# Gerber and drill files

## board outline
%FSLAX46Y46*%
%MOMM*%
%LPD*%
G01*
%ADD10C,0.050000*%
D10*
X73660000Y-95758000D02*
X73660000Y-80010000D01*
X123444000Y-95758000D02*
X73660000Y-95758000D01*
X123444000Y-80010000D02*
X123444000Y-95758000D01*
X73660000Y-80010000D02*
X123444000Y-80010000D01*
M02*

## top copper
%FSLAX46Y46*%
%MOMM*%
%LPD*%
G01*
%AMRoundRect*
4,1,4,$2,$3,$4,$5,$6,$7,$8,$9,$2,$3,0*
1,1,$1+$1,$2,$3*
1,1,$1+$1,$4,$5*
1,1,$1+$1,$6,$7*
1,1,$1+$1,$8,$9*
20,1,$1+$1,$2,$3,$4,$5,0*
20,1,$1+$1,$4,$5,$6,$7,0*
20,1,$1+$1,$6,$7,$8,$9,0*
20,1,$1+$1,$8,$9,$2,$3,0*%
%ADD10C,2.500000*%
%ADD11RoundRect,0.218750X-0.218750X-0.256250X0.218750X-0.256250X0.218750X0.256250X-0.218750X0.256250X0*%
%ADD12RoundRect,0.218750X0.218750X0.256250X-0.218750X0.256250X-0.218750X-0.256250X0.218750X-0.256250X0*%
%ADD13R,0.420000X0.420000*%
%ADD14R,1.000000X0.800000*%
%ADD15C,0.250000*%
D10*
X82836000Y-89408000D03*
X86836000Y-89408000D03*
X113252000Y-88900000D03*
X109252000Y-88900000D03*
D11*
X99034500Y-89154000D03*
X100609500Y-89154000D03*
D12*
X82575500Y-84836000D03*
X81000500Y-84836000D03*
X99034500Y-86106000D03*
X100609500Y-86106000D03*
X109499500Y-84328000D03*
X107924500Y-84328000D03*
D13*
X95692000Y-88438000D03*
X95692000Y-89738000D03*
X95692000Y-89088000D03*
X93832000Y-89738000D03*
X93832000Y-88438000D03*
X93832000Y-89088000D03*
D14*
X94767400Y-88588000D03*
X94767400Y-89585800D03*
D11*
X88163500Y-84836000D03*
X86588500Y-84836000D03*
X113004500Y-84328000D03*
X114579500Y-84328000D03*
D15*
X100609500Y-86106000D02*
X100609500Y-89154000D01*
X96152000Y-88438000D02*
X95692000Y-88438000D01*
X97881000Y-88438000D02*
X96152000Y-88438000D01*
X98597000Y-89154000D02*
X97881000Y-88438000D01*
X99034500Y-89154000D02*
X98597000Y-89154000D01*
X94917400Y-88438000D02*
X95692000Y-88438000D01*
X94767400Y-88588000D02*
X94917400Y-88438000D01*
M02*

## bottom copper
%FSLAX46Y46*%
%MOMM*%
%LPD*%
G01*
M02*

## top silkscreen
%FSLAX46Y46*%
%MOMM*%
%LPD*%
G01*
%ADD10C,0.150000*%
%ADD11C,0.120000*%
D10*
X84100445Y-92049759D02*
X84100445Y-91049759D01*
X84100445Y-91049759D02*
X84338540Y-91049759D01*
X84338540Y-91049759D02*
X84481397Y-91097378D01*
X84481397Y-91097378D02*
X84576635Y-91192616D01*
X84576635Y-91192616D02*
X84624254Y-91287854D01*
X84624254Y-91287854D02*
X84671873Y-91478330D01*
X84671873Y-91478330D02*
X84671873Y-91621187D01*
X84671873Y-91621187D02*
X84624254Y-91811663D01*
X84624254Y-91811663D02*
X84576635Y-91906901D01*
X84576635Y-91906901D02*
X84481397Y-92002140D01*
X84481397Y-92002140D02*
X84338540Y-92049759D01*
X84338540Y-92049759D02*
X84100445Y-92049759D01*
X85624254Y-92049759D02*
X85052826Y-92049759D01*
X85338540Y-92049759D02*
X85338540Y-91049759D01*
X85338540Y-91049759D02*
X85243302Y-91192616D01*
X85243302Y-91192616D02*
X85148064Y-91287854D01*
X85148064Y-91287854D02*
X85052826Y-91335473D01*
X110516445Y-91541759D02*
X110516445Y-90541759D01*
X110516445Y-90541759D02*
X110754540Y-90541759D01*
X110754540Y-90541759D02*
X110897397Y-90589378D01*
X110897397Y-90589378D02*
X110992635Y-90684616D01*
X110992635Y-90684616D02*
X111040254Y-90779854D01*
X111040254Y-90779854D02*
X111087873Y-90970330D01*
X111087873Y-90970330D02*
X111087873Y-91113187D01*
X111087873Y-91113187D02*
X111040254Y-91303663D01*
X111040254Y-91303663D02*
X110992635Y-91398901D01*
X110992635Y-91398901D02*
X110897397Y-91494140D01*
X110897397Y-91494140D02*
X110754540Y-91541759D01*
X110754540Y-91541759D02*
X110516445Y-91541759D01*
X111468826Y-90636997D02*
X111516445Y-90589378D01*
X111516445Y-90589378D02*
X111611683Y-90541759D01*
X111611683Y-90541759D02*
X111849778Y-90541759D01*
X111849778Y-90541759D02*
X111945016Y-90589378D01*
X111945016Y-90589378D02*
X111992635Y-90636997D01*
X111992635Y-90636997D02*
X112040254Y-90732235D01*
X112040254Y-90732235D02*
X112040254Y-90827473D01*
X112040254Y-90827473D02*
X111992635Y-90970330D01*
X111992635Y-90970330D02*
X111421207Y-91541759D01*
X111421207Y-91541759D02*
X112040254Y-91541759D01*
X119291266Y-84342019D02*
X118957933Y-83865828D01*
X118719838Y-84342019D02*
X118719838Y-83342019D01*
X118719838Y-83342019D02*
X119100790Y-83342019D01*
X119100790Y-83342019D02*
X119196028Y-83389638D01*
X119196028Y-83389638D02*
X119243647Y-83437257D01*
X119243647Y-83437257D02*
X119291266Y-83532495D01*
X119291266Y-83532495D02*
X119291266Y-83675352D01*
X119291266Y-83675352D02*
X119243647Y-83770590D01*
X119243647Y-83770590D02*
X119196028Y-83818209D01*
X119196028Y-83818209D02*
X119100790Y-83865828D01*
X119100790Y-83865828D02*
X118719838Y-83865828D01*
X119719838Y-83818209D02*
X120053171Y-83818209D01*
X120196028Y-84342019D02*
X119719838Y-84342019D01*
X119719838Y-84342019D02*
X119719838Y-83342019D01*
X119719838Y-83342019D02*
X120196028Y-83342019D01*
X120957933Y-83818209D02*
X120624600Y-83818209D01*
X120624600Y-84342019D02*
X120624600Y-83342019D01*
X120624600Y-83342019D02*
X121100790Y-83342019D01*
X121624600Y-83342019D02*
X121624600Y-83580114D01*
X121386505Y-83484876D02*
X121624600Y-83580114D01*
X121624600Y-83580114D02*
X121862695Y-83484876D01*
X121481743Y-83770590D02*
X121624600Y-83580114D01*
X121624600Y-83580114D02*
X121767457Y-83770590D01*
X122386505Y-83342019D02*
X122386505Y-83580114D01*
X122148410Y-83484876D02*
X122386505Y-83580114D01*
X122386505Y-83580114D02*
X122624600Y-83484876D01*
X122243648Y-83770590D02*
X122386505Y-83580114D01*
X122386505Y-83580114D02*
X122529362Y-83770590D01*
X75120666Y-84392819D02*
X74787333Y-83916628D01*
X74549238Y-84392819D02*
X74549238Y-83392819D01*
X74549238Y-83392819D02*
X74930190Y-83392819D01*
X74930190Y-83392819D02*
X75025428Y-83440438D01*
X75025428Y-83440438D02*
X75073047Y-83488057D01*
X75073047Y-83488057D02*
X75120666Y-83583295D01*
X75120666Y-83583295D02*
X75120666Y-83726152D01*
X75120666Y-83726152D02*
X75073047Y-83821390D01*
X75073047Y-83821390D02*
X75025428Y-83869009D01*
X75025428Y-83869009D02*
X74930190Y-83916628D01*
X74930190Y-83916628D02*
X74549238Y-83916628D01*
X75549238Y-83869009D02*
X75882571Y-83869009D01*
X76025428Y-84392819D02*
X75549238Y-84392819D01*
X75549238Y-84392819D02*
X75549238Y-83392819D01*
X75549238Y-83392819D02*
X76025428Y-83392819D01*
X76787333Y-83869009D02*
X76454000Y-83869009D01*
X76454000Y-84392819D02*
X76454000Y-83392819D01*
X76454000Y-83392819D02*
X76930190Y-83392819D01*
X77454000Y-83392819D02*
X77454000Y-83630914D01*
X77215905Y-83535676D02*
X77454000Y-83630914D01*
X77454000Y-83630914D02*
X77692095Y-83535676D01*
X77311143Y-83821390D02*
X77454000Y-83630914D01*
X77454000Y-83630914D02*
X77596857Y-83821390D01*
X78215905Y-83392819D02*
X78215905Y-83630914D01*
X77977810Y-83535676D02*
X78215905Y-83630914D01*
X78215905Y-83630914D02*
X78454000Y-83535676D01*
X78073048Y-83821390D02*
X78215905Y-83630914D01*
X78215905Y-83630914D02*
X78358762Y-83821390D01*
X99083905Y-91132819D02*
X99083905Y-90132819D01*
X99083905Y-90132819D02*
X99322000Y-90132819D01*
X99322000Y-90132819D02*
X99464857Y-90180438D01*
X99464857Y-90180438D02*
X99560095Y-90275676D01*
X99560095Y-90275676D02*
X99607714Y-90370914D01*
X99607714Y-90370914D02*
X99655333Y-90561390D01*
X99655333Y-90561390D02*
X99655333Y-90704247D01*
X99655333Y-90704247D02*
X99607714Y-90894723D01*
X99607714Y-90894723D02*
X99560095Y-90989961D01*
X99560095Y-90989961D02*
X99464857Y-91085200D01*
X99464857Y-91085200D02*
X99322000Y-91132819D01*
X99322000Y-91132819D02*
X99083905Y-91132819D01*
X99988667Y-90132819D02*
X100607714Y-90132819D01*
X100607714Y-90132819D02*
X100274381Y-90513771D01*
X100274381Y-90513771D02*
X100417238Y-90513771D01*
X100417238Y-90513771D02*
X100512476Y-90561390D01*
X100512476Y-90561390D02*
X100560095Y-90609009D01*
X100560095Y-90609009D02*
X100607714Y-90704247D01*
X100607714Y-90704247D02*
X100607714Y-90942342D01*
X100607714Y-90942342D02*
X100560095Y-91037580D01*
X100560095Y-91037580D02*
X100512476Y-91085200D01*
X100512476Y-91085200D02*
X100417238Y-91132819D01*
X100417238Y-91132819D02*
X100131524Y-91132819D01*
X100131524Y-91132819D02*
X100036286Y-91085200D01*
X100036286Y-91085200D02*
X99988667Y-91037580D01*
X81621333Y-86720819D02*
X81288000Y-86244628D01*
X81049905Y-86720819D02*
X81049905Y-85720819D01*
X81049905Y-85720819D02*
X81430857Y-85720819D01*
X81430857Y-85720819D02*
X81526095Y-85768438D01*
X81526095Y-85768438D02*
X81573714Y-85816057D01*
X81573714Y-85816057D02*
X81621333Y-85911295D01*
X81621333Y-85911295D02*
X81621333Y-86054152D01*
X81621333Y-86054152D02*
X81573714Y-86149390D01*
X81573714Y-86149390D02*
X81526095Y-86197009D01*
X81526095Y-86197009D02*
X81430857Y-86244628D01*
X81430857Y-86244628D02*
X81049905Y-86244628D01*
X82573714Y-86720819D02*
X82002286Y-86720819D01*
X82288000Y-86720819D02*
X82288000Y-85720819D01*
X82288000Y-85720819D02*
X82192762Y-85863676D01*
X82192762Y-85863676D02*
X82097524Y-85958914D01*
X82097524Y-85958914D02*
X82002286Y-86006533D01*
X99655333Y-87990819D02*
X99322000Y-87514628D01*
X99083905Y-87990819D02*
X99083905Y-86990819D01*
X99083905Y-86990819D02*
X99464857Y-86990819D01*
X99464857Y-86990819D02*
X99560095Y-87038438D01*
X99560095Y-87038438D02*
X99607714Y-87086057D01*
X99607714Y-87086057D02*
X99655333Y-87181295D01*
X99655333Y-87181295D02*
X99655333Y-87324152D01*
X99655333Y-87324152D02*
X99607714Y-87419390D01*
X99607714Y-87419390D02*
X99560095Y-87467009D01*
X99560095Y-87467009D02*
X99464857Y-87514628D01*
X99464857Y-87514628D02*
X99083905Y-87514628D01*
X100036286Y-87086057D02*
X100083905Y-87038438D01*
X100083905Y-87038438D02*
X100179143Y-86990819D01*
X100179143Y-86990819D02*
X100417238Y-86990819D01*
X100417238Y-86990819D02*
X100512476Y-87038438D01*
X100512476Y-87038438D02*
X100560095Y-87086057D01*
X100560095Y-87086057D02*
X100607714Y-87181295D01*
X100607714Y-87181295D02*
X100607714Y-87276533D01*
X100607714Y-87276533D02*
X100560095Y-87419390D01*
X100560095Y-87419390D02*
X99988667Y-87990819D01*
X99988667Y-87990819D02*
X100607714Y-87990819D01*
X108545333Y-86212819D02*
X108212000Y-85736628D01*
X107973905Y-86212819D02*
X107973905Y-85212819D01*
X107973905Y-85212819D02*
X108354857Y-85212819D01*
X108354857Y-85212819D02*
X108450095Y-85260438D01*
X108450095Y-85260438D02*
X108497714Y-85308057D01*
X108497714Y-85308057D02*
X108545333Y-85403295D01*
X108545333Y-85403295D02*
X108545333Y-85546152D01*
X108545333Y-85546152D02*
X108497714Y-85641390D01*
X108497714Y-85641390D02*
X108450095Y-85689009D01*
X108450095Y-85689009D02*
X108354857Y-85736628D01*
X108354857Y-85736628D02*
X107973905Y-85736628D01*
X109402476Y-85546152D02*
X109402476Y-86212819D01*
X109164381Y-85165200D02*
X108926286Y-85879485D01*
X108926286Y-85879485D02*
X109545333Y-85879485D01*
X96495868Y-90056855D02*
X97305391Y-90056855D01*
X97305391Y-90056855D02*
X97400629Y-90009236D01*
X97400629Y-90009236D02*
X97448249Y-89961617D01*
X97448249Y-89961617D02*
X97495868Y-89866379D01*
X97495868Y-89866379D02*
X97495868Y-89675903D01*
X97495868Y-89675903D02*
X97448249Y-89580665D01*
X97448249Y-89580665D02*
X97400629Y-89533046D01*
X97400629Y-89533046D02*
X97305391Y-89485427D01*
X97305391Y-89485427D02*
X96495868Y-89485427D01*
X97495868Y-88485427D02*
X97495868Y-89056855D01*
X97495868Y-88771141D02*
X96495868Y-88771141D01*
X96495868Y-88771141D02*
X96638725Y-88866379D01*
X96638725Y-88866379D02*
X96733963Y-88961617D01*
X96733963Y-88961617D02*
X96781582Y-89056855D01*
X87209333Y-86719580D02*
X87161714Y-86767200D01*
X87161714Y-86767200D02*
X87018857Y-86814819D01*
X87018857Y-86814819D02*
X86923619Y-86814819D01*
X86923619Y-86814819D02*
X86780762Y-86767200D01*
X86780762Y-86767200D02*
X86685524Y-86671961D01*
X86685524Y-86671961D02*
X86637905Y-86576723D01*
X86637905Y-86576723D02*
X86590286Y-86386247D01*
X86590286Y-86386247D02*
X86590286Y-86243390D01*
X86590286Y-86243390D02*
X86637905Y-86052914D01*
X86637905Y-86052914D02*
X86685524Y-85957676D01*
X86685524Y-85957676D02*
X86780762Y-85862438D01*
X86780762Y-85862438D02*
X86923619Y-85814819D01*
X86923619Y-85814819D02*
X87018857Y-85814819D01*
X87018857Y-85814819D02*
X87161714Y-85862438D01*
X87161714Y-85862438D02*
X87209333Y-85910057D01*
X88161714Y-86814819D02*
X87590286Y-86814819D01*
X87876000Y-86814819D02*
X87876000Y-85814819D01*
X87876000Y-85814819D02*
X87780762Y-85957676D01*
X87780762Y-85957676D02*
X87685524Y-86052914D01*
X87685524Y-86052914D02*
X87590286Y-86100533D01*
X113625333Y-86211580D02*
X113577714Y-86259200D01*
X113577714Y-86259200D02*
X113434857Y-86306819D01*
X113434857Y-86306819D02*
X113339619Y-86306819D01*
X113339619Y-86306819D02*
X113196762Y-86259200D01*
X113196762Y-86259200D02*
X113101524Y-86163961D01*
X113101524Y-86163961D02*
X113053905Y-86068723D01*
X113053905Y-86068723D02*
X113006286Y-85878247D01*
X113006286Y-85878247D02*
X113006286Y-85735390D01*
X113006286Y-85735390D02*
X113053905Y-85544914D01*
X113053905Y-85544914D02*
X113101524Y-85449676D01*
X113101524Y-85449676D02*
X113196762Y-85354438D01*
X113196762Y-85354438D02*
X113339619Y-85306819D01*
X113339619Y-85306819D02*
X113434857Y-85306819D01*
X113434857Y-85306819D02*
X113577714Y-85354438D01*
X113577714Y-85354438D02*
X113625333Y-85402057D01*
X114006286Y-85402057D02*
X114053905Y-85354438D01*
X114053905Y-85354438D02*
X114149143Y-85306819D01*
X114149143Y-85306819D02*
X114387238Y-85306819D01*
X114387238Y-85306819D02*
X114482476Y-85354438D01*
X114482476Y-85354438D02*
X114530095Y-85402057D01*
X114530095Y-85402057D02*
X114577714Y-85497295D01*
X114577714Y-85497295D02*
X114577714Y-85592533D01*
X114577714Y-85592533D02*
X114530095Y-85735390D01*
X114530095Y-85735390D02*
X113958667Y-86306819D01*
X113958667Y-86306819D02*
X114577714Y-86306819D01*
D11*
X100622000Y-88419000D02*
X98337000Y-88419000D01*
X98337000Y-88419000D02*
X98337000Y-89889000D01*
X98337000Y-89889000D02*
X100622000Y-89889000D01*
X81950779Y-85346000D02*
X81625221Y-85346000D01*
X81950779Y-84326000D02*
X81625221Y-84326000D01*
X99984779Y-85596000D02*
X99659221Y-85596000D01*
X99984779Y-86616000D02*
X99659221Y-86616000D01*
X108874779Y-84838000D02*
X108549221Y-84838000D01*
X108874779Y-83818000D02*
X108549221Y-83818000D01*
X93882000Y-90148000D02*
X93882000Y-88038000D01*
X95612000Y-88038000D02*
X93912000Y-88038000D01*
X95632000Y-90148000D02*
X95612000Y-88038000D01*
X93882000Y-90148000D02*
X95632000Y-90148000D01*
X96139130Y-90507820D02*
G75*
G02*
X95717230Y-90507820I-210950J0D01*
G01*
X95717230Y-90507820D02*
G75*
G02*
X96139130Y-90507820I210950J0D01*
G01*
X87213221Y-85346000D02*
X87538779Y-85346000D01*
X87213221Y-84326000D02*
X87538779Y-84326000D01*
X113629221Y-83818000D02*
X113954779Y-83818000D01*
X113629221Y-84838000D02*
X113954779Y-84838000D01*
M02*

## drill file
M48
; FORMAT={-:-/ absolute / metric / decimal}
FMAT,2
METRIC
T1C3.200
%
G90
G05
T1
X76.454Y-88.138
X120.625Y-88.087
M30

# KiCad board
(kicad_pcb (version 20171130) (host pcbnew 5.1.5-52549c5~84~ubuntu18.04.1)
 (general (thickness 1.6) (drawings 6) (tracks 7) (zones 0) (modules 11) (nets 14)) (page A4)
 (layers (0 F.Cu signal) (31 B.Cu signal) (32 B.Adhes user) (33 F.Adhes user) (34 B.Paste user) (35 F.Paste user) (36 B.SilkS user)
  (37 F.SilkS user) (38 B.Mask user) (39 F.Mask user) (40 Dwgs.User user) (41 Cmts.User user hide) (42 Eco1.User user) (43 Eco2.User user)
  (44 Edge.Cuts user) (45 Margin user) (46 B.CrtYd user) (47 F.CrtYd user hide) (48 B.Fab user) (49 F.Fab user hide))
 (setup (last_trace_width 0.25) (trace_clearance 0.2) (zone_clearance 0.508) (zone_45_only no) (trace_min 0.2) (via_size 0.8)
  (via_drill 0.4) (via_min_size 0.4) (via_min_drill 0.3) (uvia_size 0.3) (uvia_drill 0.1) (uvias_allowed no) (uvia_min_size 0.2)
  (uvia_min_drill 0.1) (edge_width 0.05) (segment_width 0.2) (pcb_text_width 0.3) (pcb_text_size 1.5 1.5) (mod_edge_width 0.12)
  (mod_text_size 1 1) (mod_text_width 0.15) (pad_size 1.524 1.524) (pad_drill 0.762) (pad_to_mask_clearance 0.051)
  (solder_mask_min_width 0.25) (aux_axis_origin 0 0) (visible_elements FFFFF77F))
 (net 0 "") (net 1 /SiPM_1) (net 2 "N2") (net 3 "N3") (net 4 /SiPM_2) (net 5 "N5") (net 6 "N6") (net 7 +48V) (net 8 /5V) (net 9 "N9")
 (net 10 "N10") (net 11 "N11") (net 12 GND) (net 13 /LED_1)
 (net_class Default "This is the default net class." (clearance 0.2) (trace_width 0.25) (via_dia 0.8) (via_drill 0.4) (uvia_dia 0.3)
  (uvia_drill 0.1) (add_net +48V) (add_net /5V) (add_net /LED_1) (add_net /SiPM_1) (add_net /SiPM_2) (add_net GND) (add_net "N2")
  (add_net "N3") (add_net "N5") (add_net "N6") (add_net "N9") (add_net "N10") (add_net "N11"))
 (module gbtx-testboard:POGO (layer F.Cu) (at 84.836 89.408)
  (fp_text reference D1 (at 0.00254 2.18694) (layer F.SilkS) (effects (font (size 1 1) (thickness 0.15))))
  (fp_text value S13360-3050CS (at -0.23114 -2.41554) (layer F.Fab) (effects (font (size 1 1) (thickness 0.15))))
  (pad 1 smd circle (at -2 0) (size 2.5 2.5) (layers F.Cu F.Paste F.Mask) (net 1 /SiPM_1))
  (pad 2 smd circle (at 2 0) (size 2.5 2.5) (layers F.Cu F.Paste F.Mask) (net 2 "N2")))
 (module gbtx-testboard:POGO (layer F.Cu) (at 111.252 88.9)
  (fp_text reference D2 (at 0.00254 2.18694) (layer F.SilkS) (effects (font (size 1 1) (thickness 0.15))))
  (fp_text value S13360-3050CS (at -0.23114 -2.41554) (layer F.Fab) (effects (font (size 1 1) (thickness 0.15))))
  (pad 2 smd circle (at 2 0) (size 2.5 2.5) (layers F.Cu F.Paste F.Mask) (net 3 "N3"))
  (pad 1 smd circle (at -2 0) (size 2.5 2.5) (layers F.Cu F.Paste F.Mask) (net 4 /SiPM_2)))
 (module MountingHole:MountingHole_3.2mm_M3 (layer F.Cu) (at 120.6246 88.0872)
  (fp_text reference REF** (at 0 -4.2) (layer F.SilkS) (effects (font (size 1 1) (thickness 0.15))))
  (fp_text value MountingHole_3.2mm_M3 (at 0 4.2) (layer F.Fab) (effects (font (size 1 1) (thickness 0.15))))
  (pad 1 np_thru_hole circle (at 0 0) (size 3.2 3.2) (drill 3.2) (layers *.Cu *.Mask)))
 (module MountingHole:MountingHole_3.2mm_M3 (layer F.Cu) (at 76.454 88.138)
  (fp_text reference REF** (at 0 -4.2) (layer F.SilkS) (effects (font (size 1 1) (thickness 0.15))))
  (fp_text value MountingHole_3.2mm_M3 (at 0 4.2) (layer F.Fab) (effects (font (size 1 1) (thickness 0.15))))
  (pad 1 np_thru_hole circle (at 0 0) (size 3.2 3.2) (drill 3.2) (layers *.Cu *.Mask)))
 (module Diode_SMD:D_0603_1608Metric (layer F.Cu) (at 99.822 89.154)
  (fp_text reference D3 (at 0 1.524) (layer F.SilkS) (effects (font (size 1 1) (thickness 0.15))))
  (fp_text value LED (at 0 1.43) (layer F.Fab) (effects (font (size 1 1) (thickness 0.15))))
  (fp_line (start 0.8 -0.735) (end -1.485 -0.735) (layer F.SilkS) (width 0.12))
  (fp_line (start -1.485 -0.735) (end -1.485 0.735) (layer F.SilkS) (width 0.12))
  (fp_line (start -1.485 0.735) (end 0.8 0.735) (layer F.SilkS) (width 0.12))
  (pad 1 smd roundrect (at -0.7875 0) (size 0.875 0.95) (layers F.Cu F.Paste F.Mask) (roundrect_rratio 0.25) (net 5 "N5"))
  (pad 2 smd roundrect (at 0.7875 0) (size 0.875 0.95) (layers F.Cu F.Paste F.Mask) (roundrect_rratio 0.25) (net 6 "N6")))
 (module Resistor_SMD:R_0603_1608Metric (layer F.Cu) (at 81.788 84.836 180)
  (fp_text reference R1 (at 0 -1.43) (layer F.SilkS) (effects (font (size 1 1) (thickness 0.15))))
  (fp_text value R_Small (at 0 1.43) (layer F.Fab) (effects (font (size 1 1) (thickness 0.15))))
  (fp_line (start -0.162779 -0.51) (end 0.162779 -0.51) (layer F.SilkS) (width 0.12))
  (fp_line (start -0.162779 0.51) (end 0.162779 0.51) (layer F.SilkS) (width 0.12))
  (pad 1 smd roundrect (at -0.7875 0 180) (size 0.875 0.95) (layers F.Cu F.Paste F.Mask) (roundrect_rratio 0.25) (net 2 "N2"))
  (pad 2 smd roundrect (at 0.7875 0 180) (size 0.875 0.95) (layers F.Cu F.Paste F.Mask) (roundrect_rratio 0.25) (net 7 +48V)))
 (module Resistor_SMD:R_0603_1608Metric (layer F.Cu) (at 99.822 86.106 180)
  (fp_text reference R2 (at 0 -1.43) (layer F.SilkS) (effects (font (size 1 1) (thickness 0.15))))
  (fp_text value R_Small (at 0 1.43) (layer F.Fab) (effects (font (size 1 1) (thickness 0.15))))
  (fp_line (start -0.162779 0.51) (end 0.162779 0.51) (layer F.SilkS) (width 0.12))
  (fp_line (start -0.162779 -0.51) (end 0.162779 -0.51) (layer F.SilkS) (width 0.12))
  (pad 2 smd roundrect (at 0.7875 0 180) (size 0.875 0.95) (layers F.Cu F.Paste F.Mask) (roundrect_rratio 0.25) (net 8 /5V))
  (pad 1 smd roundrect (at -0.7875 0 180) (size 0.875 0.95) (layers F.Cu F.Paste F.Mask) (roundrect_rratio 0.25) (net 6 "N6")))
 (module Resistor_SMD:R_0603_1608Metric (layer F.Cu) (at 108.712 84.328 180)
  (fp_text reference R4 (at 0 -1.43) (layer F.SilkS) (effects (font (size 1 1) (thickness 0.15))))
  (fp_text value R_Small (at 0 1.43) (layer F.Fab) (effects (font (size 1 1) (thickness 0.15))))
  (fp_line (start -0.162779 -0.51) (end 0.162779 -0.51) (layer F.SilkS) (width 0.12))
  (fp_line (start -0.162779 0.51) (end 0.162779 0.51) (layer F.SilkS) (width 0.12))
  (pad 1 smd roundrect (at -0.7875 0 180) (size 0.875 0.95) (layers F.Cu F.Paste F.Mask) (roundrect_rratio 0.25) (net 3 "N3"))
  (pad 2 smd roundrect (at 0.7875 0 180) (size 0.875 0.95) (layers F.Cu F.Paste F.Mask) (roundrect_rratio 0.25) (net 7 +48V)))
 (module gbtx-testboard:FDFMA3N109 (layer F.Cu) (at 94.742 88.138 90)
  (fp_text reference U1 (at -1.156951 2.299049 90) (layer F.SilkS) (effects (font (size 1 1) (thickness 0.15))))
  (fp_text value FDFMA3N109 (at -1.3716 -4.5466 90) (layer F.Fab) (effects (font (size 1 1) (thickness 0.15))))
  (fp_line (start -2.01 -0.86) (end 0.1 -0.86) (layer F.SilkS) (width 0.12))
  (fp_line (start 0.1 0.87) (end 0.1 -0.83) (layer F.SilkS) (width 0.12))
  (fp_line (start -2.01 0.89) (end 0.1 0.87) (layer F.SilkS) (width 0.12))
  (fp_line (start -2.01 -0.86) (end -2.01 0.89) (layer F.SilkS) (width 0.12))
  (fp_circle (center -2.36982 1.18618) (end -2.18982 1.29618) (layer F.SilkS) (width 0.12))
  (pad 3 smd rect (at -0.3 0.95 90) (size 0.42 0.42) (layers F.Cu F.Paste F.Mask) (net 5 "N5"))
  (pad 1 smd rect (at -1.6 0.95 90) (size 0.42 0.42) (layers F.Cu F.Paste F.Mask) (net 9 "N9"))
  (pad 2 smd rect (at -0.95 0.95 90) (size 0.42 0.42) (layers F.Cu F.Paste F.Mask) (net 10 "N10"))
  (pad 6 smd rect (at -1.6 -0.91 90) (size 0.42 0.42) (layers F.Cu F.Paste F.Mask) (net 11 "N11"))
  (pad 4 smd rect (at -0.3 -0.91 90) (size 0.42 0.42) (layers F.Cu F.Paste F.Mask) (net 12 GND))
  (pad 5 smd rect (at -0.95 -0.91 90) (size 0.42 0.42) (layers F.Cu F.Paste F.Mask) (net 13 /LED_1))
  (pad 3 smd rect (at -0.45 0.0254 90) (size 0.8 1) (layers F.Cu F.Paste F.Mask) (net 5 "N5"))
  (pad K smd rect (at -1.4478 0.0254 90) (size 0.8 1) (layers F.Cu F.Paste F.Mask)))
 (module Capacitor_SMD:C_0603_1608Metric (layer F.Cu) (at 87.376 84.836)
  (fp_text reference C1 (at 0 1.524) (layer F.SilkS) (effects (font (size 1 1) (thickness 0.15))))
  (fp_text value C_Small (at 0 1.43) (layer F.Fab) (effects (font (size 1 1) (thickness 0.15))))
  (fp_line (start -0.162779 0.51) (end 0.162779 0.51) (layer F.SilkS) (width 0.12))
  (fp_line (start -0.162779 -0.51) (end 0.162779 -0.51) (layer F.SilkS) (width 0.12))
  (pad 2 smd roundrect (at 0.7875 0) (size 0.875 0.95) (layers F.Cu F.Paste F.Mask) (roundrect_rratio 0.25) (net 12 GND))
  (pad 1 smd roundrect (at -0.7875 0) (size 0.875 0.95) (layers F.Cu F.Paste F.Mask) (roundrect_rratio 0.25) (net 2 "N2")))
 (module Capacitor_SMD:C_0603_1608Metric (layer F.Cu) (at 113.792 84.328)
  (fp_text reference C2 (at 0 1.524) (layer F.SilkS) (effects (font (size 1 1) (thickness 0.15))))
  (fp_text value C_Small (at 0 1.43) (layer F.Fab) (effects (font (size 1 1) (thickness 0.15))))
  (fp_line (start -0.162779 -0.51) (end 0.162779 -0.51) (layer F.SilkS) (width 0.12))
  (fp_line (start -0.162779 0.51) (end 0.162779 0.51) (layer F.SilkS) (width 0.12))
  (pad 1 smd roundrect (at -0.7875 0) (size 0.875 0.95) (layers F.Cu F.Paste F.Mask) (roundrect_rratio 0.25) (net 3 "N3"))
  (pad 2 smd roundrect (at 0.7875 0) (size 0.875 0.95) (layers F.Cu F.Paste F.Mask) (roundrect_rratio 0.25) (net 12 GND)))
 (gr_line (start 73.66 95.758) (end 73.66 80.01) (layer Edge.Cuts) (width 0.05))
 (gr_line (start 123.444 95.758) (end 73.66 95.758) (layer Edge.Cuts) (width 0.05))
 (gr_line (start 123.444 80.01) (end 123.444 95.758) (layer Edge.Cuts) (width 0.05))
 (gr_line (start 73.66 80.01) (end 123.444 80.01) (layer Edge.Cuts) (width 0.05))
 (segment (start 100.6095 86.106) (end 100.6095 89.154) (width 0.25) (layer F.Cu) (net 6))
 (segment (start 96.152 88.438) (end 95.692 88.438) (width 0.25) (layer F.Cu) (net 5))
 (segment (start 97.881 88.438) (end 96.152 88.438) (width 0.25) (layer F.Cu) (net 5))
 (segment (start 98.597 89.154) (end 97.881 88.438) (width 0.25) (layer F.Cu) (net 5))
 (segment (start 99.0345 89.154) (end 98.597 89.154) (width 0.25) (layer F.Cu) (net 5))
 (segment (start 94.9174 88.438) (end 95.692 88.438) (width 0.25) (layer F.Cu) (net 5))
 (segment (start 94.7674 88.588) (end 94.9174 88.438) (width 0.25) (layer F.Cu) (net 5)))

